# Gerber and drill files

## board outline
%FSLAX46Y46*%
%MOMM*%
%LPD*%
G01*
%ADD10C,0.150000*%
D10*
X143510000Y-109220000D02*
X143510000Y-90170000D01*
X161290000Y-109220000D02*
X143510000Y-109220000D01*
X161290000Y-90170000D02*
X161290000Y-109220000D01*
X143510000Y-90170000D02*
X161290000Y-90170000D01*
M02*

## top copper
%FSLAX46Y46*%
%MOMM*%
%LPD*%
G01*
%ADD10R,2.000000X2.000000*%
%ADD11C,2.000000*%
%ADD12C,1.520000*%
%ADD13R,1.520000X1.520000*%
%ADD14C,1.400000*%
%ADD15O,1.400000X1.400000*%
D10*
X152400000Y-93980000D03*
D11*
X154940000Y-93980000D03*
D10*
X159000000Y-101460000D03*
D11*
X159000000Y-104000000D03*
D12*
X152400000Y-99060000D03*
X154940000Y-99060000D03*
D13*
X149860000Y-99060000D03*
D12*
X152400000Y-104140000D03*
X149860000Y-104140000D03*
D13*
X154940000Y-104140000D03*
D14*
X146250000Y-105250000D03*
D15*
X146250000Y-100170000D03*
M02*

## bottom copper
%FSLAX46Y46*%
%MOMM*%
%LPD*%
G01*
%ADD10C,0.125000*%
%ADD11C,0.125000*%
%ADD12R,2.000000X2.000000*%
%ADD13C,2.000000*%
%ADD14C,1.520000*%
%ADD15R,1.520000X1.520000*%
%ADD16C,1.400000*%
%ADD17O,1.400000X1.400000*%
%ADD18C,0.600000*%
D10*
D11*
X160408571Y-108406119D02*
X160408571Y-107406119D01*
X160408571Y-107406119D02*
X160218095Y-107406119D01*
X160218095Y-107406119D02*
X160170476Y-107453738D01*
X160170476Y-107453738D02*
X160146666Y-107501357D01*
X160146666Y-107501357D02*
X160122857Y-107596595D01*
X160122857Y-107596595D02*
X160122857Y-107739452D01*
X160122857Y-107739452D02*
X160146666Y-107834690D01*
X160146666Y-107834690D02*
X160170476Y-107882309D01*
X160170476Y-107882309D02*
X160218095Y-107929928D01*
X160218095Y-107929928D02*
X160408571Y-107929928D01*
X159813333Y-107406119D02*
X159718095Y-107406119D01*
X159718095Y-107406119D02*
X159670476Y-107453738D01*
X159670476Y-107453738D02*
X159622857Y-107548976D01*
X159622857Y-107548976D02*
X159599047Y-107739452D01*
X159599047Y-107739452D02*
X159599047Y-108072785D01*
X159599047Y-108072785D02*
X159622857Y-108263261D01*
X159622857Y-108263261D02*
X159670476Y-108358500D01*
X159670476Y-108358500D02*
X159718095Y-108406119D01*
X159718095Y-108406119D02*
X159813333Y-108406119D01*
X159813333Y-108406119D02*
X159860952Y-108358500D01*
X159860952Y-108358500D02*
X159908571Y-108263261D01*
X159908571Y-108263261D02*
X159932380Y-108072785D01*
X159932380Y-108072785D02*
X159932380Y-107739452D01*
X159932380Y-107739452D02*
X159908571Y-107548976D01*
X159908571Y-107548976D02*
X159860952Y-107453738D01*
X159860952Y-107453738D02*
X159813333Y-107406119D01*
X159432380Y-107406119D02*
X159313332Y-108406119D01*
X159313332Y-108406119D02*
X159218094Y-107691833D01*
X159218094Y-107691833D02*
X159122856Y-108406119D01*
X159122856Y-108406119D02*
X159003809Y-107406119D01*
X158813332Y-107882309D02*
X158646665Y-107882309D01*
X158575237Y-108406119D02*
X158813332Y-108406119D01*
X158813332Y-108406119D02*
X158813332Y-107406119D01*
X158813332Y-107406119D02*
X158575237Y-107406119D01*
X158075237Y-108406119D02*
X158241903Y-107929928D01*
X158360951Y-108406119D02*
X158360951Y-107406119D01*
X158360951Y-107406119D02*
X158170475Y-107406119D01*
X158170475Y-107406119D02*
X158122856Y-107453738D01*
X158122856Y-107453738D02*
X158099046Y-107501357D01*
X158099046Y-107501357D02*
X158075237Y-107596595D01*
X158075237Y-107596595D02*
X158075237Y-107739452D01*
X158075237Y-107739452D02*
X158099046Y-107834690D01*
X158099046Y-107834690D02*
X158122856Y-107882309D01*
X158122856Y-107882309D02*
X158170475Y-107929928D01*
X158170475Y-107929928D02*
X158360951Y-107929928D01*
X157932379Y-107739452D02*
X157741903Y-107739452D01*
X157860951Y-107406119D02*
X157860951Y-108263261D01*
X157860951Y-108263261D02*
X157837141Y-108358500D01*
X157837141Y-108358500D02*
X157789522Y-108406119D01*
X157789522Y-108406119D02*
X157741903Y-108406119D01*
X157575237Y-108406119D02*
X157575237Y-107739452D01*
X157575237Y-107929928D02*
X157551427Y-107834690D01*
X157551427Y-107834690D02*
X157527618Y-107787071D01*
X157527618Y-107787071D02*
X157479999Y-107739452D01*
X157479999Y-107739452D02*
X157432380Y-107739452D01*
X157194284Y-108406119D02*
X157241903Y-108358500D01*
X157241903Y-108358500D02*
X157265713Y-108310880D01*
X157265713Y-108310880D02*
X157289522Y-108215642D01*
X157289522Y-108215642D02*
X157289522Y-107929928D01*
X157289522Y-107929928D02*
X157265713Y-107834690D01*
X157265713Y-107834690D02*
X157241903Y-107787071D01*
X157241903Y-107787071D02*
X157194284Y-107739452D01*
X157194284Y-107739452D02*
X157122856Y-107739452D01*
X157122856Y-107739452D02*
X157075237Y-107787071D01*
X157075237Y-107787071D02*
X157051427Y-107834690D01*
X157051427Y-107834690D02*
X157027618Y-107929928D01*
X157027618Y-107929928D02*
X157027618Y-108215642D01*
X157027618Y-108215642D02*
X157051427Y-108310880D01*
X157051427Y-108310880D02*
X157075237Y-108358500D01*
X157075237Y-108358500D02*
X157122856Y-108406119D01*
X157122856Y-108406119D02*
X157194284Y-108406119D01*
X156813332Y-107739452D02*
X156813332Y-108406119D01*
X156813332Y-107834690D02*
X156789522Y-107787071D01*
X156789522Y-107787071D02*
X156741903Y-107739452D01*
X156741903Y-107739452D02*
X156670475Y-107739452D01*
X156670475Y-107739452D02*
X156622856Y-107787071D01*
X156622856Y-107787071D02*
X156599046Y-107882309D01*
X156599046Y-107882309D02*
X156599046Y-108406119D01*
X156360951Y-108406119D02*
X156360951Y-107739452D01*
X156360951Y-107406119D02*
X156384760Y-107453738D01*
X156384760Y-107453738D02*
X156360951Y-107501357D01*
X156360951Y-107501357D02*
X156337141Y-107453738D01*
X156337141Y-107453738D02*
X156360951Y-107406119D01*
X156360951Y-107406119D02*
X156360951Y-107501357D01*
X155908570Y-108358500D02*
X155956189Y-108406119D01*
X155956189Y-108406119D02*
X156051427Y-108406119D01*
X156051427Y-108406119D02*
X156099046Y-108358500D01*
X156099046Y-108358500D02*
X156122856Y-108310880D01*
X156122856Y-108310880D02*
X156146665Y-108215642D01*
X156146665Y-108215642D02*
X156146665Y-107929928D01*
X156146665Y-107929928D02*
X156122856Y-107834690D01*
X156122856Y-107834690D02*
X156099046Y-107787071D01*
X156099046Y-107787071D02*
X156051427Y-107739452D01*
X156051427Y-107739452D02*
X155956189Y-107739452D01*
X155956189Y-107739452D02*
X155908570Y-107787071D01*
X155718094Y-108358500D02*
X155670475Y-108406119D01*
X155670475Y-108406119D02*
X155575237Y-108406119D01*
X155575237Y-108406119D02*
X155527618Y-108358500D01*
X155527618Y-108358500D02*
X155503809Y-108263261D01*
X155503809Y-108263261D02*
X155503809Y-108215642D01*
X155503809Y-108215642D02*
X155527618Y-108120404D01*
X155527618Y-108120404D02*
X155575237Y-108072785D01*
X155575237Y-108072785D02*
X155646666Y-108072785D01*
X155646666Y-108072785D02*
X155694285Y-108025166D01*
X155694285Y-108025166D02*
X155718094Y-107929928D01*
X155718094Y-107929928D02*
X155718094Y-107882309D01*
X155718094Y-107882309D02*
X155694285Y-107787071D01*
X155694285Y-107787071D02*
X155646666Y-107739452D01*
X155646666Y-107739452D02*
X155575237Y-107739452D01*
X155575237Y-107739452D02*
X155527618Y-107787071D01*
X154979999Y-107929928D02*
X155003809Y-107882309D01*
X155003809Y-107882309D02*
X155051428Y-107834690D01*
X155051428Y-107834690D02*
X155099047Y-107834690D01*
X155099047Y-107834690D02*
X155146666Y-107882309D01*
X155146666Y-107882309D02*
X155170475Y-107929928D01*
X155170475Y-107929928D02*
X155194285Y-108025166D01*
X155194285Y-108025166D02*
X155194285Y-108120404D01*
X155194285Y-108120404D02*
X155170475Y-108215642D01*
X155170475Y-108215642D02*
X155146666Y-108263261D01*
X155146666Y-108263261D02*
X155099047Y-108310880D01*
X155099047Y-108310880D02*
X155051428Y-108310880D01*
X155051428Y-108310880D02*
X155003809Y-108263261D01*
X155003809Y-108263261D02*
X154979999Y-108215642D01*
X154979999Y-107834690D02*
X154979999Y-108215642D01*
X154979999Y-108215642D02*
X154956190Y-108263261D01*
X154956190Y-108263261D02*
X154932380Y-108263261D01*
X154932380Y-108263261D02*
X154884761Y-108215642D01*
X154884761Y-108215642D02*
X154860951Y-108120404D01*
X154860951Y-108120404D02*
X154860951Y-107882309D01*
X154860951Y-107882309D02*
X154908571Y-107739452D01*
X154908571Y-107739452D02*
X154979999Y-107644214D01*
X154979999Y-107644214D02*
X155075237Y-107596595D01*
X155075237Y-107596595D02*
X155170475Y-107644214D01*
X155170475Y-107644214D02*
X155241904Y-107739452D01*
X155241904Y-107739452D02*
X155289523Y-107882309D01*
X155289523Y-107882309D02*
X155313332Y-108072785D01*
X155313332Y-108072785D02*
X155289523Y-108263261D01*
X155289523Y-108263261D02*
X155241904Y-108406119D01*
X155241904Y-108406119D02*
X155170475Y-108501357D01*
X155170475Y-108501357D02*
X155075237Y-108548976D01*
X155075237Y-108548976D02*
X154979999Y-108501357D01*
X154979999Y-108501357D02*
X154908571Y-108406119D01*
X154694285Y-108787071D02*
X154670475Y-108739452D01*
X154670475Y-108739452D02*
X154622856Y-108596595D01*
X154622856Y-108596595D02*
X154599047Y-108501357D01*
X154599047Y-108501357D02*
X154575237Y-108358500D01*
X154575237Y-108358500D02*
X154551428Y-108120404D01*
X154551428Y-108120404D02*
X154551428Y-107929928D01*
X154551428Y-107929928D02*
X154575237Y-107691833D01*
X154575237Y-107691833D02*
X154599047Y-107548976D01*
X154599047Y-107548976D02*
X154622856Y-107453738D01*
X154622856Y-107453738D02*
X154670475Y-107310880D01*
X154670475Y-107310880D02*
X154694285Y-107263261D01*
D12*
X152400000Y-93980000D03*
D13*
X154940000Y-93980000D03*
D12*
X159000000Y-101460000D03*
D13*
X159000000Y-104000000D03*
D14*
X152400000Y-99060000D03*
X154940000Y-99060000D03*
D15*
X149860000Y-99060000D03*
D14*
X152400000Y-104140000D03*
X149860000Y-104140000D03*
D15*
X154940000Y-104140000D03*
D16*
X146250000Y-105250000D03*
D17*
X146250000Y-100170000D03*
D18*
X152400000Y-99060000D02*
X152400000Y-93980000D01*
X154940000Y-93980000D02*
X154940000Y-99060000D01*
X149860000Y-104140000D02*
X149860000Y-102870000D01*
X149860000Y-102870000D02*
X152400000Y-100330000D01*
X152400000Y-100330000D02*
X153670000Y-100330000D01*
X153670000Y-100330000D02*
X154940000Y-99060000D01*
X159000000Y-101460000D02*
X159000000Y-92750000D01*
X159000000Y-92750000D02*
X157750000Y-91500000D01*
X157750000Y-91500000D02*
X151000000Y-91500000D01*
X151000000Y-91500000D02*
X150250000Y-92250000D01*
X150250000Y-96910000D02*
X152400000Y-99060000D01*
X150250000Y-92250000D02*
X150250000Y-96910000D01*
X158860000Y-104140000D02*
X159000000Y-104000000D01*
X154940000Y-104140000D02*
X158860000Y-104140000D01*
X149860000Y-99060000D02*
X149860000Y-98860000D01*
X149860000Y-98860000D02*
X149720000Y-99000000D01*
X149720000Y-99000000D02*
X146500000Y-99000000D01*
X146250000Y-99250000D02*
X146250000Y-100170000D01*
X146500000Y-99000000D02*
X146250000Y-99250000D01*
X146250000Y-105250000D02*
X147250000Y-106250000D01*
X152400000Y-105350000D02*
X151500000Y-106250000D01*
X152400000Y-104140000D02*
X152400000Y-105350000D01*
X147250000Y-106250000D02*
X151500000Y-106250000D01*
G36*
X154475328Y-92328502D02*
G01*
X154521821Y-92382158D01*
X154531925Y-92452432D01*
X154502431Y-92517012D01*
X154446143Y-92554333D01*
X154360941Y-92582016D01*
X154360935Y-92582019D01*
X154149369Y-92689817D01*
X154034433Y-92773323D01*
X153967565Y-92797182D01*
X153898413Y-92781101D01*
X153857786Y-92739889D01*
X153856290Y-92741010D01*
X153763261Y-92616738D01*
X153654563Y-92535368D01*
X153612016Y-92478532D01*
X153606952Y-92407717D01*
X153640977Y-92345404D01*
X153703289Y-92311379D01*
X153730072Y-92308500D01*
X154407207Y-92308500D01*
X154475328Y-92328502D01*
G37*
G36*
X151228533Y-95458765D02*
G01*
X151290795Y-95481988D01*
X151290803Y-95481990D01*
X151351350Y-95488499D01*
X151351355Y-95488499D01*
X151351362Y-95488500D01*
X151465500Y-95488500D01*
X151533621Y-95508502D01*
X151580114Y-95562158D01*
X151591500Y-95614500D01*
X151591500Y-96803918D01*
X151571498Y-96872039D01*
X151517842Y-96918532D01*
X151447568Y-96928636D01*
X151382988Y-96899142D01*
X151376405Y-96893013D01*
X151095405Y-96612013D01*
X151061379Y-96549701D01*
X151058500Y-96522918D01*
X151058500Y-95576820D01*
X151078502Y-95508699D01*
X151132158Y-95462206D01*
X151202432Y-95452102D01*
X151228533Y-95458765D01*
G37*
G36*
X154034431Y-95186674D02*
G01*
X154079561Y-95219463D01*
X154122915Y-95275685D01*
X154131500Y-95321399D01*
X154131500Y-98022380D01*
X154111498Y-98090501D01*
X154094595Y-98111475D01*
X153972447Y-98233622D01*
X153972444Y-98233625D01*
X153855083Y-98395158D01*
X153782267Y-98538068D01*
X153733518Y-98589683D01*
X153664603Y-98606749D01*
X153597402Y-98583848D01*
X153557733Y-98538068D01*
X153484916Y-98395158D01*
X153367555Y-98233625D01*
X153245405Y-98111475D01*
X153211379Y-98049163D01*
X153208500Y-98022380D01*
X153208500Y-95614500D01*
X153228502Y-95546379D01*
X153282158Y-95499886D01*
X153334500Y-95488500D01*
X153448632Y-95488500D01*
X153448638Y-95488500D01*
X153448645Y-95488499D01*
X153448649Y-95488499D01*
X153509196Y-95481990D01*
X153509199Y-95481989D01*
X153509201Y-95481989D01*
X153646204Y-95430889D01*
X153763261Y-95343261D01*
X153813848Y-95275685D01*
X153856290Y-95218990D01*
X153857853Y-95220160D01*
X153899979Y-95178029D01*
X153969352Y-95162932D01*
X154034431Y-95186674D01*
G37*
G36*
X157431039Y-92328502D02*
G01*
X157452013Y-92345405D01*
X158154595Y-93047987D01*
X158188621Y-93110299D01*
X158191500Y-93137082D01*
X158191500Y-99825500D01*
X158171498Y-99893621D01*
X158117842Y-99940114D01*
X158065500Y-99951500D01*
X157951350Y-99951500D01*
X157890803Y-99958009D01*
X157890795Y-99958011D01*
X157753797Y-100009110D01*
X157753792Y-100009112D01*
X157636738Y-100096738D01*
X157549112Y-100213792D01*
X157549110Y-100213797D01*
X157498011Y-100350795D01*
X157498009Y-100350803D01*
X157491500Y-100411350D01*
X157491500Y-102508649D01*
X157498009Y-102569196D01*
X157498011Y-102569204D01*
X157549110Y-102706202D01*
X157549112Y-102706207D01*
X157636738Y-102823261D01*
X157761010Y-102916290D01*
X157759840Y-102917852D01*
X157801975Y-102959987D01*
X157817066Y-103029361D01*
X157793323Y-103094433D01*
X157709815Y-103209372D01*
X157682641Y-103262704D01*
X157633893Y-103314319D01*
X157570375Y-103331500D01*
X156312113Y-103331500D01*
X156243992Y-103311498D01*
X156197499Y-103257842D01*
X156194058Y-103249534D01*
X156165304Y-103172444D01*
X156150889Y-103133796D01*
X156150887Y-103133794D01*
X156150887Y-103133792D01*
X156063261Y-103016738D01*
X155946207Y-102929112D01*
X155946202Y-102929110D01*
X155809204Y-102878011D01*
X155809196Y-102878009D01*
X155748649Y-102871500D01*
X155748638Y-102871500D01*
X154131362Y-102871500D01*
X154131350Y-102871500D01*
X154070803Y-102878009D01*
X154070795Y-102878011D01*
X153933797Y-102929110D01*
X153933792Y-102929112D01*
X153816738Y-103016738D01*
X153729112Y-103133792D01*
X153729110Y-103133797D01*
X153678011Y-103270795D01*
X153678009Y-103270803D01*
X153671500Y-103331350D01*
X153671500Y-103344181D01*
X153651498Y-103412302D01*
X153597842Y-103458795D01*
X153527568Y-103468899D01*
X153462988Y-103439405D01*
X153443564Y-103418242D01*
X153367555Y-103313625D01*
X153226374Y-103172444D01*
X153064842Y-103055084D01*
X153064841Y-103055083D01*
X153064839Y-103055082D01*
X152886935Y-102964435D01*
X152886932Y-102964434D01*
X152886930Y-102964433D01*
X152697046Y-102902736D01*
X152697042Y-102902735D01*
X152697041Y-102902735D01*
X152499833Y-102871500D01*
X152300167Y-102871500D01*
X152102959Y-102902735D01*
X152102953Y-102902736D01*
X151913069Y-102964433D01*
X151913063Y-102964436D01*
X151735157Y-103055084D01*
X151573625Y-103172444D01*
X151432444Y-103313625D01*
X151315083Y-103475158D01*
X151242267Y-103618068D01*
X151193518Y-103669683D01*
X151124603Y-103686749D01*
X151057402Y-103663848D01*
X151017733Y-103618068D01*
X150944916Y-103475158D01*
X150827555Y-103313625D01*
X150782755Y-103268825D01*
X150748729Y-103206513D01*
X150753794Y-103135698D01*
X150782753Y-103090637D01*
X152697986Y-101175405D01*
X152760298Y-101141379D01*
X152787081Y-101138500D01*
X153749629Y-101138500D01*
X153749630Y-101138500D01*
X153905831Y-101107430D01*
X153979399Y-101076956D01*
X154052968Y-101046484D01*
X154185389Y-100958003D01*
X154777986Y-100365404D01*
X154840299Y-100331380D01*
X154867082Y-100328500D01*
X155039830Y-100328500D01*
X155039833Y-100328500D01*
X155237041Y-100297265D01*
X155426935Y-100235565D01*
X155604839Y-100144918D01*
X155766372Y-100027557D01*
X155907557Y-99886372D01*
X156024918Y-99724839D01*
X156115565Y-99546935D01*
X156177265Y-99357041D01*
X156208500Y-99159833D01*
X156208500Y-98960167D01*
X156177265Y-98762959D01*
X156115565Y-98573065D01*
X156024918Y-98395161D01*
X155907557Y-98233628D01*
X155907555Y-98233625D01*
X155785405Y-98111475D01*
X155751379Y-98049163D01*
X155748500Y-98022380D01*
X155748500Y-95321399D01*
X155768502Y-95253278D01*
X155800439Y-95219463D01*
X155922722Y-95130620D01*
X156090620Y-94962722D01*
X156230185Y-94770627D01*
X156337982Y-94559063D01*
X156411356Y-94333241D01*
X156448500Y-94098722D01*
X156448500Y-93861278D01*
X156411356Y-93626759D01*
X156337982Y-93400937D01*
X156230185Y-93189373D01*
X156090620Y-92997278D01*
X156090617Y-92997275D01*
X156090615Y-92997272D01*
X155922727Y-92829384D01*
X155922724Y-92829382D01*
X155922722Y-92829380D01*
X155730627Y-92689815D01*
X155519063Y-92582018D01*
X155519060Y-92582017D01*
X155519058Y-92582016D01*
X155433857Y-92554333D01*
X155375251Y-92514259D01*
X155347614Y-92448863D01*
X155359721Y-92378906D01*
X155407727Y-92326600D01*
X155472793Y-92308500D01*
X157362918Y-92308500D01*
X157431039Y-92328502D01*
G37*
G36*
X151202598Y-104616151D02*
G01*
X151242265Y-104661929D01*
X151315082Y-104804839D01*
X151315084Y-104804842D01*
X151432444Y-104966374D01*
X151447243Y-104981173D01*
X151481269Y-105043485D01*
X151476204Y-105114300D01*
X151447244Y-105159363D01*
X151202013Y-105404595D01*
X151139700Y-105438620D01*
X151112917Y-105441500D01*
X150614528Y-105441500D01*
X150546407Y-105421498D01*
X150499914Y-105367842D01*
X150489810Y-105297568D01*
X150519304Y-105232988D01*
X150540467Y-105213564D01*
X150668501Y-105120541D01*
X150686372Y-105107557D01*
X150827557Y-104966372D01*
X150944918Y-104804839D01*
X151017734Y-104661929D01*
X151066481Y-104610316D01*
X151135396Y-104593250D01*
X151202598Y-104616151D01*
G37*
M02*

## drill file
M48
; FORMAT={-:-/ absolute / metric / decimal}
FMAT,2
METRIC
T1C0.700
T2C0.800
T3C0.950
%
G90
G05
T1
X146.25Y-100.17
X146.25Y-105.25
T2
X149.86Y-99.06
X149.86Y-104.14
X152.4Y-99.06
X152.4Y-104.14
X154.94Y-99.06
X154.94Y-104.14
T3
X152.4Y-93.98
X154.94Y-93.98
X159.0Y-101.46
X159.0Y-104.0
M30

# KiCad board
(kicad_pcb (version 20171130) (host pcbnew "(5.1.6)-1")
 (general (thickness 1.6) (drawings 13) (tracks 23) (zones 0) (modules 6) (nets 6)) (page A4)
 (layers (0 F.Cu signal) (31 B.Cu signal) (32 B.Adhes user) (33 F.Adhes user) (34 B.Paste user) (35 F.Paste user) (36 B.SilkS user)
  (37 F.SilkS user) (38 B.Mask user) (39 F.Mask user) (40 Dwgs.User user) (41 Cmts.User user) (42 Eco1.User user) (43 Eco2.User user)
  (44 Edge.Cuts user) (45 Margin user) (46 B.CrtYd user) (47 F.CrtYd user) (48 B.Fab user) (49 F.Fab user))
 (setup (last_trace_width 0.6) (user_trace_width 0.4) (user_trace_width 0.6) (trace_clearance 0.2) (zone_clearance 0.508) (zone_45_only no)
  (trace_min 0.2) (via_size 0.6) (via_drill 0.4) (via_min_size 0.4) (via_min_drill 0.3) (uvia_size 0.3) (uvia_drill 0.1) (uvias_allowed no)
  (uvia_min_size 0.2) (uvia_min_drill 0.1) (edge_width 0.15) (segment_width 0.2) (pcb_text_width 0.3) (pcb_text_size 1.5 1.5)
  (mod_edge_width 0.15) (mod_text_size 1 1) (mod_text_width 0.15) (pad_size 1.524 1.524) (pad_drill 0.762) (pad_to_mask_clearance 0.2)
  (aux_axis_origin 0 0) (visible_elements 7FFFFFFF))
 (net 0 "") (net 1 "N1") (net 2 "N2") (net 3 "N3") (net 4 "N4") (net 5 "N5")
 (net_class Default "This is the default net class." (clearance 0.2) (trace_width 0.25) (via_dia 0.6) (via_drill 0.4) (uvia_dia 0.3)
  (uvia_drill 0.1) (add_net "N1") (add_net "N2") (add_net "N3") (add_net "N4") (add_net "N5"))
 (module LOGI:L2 (layer F.Cu) (at 146.75 94.25)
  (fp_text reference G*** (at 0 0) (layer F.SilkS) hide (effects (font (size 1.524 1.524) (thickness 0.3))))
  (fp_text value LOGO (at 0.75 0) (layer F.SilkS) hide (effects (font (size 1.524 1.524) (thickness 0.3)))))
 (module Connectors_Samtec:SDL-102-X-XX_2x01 (layer F.Cu) (at 152.4 93.98)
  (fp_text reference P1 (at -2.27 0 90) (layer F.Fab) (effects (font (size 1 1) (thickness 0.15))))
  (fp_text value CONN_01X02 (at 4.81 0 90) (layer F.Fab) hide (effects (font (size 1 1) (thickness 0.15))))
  (pad 1 thru_hole rect (at 0 0) (size 2 2) (drill 0.95) (layers *.Cu *.Mask) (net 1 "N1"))
  (pad 2 thru_hole circle (at 2.54 0) (size 2 2) (drill 0.95) (layers *.Cu *.Mask) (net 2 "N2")))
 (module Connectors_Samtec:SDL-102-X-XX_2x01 (layer F.Cu) (at 159 101.46 270)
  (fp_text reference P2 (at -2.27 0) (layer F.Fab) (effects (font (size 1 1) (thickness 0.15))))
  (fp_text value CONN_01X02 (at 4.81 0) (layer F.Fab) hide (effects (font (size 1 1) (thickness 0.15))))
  (pad 1 thru_hole rect (at 0 0 270) (size 2 2) (drill 0.95) (layers *.Cu *.Mask) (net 1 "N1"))
  (pad 2 thru_hole circle (at 2.54 0 270) (size 2 2) (drill 0.95) (layers *.Cu *.Mask) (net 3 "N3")))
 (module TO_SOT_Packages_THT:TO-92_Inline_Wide (layer F.Cu) (at 149.86 99.06)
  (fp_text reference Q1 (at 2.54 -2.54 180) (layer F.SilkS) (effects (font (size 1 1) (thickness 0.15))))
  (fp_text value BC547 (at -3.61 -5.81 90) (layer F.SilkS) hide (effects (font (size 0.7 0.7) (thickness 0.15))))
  (pad 2 thru_hole circle (at 2.54 0 90) (size 1.52 1.52) (drill 0.8) (layers *.Cu *.Mask) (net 1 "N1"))
  (pad 3 thru_hole circle (at 5.08 0 90) (size 1.52 1.52) (drill 0.8) (layers *.Cu *.Mask) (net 2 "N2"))
  (pad 1 thru_hole rect (at 0 0 90) (size 1.52 1.52) (drill 0.8) (layers *.Cu *.Mask) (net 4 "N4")))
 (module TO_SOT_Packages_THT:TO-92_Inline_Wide (layer F.Cu) (at 154.94 104.14 180)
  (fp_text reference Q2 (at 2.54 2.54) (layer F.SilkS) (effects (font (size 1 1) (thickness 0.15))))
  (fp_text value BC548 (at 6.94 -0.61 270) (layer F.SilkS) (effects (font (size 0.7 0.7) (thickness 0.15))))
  (pad 2 thru_hole circle (at 2.54 0 270) (size 1.52 1.52) (drill 0.8) (layers *.Cu *.Mask) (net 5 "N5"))
  (pad 3 thru_hole circle (at 5.08 0 270) (size 1.52 1.52) (drill 0.8) (layers *.Cu *.Mask) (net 2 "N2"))
  (pad 1 thru_hole rect (at 0 0 270) (size 1.52 1.52) (drill 0.8) (layers *.Cu *.Mask) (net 3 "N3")))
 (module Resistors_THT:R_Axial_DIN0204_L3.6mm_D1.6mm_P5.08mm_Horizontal (layer F.Cu) (at 146.25 105.25 90)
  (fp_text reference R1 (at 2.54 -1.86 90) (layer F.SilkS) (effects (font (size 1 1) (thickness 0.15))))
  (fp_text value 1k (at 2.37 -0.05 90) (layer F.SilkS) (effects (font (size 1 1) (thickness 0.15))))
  (pad 1 thru_hole circle (at 0 0 90) (size 1.4 1.4) (drill 0.7) (layers *.Cu *.Mask) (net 5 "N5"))
  (pad 2 thru_hole oval (at 5.08 0 90) (size 1.4 1.4) (drill 0.7) (layers *.Cu *.Mask) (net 4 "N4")))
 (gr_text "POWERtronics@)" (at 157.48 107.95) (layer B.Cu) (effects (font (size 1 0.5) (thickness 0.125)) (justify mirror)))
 (gr_line (start 143.51 109.22) (end 143.51 90.17) (angle 90) (layer Edge.Cuts) (width 0.15))
 (gr_line (start 161.29 109.22) (end 143.51 109.22) (angle 90) (layer Edge.Cuts) (width 0.15))
 (gr_line (start 161.29 90.17) (end 161.29 109.22) (angle 90) (layer Edge.Cuts) (width 0.15))
 (gr_line (start 143.51 90.17) (end 161.29 90.17) (angle 90) (layer Edge.Cuts) (width 0.15))
 (segment (start 152.4 99.06) (end 152.4 93.98) (width 0.6) (layer B.Cu) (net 1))
 (segment (start 154.94 93.98) (end 154.94 99.06) (width 0.6) (layer B.Cu) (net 2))
 (segment (start 149.86 104.14) (end 149.86 102.87) (width 0.6) (layer B.Cu) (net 2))
 (segment (start 149.86 102.87) (end 152.4 100.33) (width 0.6) (layer B.Cu) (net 2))
 (segment (start 152.4 100.33) (end 153.67 100.33) (width 0.6) (layer B.Cu) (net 2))
 (segment (start 153.67 100.33) (end 154.94 99.06) (width 0.6) (layer B.Cu) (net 2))
 (segment (start 159 101.46) (end 159 92.75) (width 0.6) (layer B.Cu) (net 1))
 (segment (start 159 92.75) (end 157.75 91.5) (width 0.6) (layer B.Cu) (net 1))
 (segment (start 157.75 91.5) (end 151 91.5) (width 0.6) (layer B.Cu) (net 1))
 (segment (start 151 91.5) (end 150.25 92.25) (width 0.6) (layer B.Cu) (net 1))
 (segment (start 150.25 96.91) (end 152.4 99.06) (width 0.6) (layer B.Cu) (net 1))
 (segment (start 150.25 92.25) (end 150.25 96.91) (width 0.6) (layer B.Cu) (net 1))
 (segment (start 158.86 104.14) (end 159 104) (width 0.6) (layer B.Cu) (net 3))
 (segment (start 154.94 104.14) (end 158.86 104.14) (width 0.6) (layer B.Cu) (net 3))
 (segment (start 149.86 99.06) (end 149.86 98.86) (width 0.6) (layer B.Cu) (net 4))
 (segment (start 149.86 98.86) (end 149.72 99) (width 0.6) (layer B.Cu) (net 4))
 (segment (start 149.72 99) (end 146.5 99) (width 0.6) (layer B.Cu) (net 4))
 (segment (start 146.25 99.25) (end 146.25 100.17) (width 0.6) (layer B.Cu) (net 4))
 (segment (start 146.5 99) (end 146.25 99.25) (width 0.6) (layer B.Cu) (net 4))
 (segment (start 146.25 105.25) (end 147.25 106.25) (width 0.6) (layer B.Cu) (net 5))
 (segment (start 152.4 105.35) (end 151.5 106.25) (width 0.6) (layer B.Cu) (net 5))
 (segment (start 152.4 104.14) (end 152.4 105.35) (width 0.6) (layer B.Cu) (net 5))
 (segment (start 147.25 106.25) (end 151.5 106.25) (width 0.6) (layer B.Cu) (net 5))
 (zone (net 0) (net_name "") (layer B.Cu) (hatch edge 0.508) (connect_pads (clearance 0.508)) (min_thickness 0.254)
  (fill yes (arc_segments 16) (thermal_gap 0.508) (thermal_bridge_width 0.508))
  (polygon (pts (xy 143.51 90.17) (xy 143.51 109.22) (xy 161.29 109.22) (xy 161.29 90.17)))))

